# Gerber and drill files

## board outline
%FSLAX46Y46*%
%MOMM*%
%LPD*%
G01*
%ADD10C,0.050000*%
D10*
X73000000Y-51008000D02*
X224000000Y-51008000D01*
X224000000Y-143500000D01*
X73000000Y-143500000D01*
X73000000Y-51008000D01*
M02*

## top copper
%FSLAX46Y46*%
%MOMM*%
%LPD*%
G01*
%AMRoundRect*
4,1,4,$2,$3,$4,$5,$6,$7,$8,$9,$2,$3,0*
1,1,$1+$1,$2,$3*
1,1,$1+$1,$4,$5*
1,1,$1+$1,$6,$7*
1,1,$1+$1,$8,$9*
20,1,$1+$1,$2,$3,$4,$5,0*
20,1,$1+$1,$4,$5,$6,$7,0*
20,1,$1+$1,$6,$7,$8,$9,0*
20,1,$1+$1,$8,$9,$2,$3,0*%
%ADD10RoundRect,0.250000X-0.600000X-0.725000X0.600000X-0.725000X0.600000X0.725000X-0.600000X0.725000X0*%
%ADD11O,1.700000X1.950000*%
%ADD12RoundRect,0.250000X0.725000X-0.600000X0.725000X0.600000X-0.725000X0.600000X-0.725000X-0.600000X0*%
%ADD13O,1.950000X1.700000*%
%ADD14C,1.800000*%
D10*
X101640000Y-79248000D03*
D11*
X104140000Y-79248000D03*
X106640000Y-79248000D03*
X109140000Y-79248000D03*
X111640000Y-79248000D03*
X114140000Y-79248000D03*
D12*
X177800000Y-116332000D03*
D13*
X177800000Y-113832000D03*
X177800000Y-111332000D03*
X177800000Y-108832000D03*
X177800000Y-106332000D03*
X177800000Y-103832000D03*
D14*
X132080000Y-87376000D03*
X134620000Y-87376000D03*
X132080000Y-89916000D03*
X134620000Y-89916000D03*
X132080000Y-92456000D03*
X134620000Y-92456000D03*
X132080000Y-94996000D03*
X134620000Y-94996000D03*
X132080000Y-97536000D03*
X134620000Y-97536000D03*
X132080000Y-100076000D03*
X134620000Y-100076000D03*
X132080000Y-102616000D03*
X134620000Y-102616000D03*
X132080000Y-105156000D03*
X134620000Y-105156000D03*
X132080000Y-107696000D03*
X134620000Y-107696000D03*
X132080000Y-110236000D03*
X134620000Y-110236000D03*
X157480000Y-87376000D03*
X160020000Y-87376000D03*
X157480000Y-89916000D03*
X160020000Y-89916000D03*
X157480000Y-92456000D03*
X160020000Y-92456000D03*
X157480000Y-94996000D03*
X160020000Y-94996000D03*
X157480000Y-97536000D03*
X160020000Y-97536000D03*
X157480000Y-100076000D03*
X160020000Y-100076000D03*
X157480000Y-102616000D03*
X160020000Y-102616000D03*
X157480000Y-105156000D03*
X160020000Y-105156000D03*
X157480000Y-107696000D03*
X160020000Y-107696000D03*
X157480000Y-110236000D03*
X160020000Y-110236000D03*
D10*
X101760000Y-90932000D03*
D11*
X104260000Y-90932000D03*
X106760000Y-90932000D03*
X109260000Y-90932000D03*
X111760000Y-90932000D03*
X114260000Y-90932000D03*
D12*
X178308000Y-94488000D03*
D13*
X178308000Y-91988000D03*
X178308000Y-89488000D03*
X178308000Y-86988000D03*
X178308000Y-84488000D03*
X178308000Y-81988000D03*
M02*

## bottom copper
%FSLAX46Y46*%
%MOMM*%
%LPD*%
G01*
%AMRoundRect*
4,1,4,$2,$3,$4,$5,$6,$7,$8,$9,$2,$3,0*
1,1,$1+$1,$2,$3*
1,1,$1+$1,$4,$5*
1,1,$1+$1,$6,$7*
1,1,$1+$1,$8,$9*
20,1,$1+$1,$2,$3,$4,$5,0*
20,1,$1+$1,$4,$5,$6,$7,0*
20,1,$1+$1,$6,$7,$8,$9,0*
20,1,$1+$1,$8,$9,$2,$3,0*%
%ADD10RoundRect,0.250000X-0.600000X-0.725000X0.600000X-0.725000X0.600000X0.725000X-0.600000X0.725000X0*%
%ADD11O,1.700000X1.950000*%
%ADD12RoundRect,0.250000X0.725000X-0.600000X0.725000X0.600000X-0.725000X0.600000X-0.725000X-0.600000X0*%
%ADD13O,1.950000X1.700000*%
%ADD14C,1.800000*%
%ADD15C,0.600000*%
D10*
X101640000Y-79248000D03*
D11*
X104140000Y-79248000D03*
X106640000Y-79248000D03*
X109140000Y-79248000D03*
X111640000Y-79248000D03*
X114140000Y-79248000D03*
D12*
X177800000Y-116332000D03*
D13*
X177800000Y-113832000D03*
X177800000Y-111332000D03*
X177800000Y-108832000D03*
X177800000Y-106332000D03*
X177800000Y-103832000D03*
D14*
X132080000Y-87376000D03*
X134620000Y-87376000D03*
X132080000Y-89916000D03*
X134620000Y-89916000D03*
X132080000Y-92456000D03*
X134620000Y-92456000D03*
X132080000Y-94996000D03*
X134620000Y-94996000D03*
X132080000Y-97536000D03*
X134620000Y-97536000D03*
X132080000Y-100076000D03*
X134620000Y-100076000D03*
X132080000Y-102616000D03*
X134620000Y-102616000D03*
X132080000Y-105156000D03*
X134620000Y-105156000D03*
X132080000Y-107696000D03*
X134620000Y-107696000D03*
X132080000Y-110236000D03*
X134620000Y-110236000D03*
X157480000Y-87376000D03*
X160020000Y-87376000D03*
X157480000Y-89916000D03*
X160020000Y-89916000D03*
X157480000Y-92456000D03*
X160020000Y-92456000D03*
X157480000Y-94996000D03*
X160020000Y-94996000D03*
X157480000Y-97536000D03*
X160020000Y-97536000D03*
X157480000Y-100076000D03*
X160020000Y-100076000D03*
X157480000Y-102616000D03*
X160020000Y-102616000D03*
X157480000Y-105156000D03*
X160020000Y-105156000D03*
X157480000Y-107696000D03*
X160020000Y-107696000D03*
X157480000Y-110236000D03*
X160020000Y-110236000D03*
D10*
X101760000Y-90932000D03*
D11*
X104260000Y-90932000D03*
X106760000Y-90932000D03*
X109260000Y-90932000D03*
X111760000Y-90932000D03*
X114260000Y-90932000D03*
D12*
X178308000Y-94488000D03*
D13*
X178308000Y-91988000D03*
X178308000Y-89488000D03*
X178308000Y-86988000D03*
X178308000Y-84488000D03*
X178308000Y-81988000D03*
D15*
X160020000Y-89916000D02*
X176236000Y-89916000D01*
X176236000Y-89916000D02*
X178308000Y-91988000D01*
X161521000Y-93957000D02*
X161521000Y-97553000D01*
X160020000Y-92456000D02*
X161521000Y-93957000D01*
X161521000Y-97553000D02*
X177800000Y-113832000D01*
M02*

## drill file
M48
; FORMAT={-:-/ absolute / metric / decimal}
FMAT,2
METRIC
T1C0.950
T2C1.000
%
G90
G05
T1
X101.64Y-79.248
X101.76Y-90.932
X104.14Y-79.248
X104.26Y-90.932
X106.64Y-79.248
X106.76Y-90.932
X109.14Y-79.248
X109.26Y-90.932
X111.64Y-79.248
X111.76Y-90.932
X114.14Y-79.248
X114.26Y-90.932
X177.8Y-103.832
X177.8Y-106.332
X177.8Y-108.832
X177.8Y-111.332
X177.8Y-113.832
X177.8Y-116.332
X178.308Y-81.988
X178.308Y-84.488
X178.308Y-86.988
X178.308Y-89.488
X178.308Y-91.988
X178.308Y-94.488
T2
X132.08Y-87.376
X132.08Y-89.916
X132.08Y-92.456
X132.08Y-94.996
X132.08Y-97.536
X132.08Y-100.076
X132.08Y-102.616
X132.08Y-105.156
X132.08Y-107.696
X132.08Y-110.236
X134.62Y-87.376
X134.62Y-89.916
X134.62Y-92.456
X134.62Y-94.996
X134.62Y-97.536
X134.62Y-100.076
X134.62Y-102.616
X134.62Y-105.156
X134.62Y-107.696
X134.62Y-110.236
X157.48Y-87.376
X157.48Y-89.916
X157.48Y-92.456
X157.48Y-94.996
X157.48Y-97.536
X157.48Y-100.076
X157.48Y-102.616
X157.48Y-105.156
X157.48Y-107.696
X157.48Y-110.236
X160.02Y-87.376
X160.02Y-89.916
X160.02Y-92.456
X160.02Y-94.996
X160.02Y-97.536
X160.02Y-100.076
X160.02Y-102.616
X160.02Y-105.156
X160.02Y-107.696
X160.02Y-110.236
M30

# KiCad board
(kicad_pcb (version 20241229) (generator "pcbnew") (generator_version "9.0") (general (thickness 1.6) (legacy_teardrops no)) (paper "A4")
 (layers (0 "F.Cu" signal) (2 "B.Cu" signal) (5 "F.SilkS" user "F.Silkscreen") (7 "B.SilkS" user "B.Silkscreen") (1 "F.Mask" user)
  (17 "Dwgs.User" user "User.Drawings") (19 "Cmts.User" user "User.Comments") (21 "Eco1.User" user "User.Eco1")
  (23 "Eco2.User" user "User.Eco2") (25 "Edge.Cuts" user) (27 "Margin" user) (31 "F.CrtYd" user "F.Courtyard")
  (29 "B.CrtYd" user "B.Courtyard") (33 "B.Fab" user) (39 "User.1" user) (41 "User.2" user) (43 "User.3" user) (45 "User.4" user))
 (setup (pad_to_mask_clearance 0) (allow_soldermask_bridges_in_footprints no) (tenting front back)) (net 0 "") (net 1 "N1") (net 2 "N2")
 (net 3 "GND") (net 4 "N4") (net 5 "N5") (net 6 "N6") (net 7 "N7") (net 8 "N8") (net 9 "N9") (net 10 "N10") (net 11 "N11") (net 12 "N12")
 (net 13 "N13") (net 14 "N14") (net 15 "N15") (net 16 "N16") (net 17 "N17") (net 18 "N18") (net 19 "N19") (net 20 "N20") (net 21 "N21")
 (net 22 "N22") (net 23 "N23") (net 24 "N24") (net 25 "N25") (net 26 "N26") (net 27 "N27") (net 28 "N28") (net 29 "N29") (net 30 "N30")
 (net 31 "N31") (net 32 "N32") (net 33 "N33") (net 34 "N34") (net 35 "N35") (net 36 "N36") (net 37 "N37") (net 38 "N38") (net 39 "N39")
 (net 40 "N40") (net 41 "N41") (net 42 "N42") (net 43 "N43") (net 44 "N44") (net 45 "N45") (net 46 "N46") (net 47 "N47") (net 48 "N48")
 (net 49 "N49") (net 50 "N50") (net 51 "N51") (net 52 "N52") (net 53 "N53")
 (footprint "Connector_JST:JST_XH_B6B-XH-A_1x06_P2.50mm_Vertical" (layer "F.Cu") (at 101.64 79.248)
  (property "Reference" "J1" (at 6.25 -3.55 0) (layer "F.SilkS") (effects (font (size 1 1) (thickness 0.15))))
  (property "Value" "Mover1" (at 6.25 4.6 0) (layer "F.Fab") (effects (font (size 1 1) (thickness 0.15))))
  (pad "1" thru_hole roundrect (at 0 0) (size 1.7 1.95) (drill 0.95) (layers "*.Cu" "*.Mask") (remove_unused_layers no)
   (roundrect_rratio 0.147059) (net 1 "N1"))
  (pad "2" thru_hole oval (at 2.5 0) (size 1.7 1.95) (drill 0.95) (layers "*.Cu" "*.Mask") (remove_unused_layers no) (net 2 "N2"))
  (pad "3" thru_hole oval (at 5 0) (size 1.7 1.95) (drill 0.95) (layers "*.Cu" "*.Mask") (remove_unused_layers no) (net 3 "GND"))
  (pad "4" thru_hole oval (at 7.5 0) (size 1.7 1.95) (drill 0.95) (layers "*.Cu" "*.Mask") (remove_unused_layers no) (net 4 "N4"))
  (pad "5" thru_hole oval (at 10 0) (size 1.7 1.95) (drill 0.95) (layers "*.Cu" "*.Mask") (remove_unused_layers no) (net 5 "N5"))
  (pad "6" thru_hole oval (at 12.5 0) (size 1.7 1.95) (drill 0.95) (layers "*.Cu" "*.Mask") (remove_unused_layers no) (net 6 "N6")))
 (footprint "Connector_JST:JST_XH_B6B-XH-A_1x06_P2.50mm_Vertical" (layer "F.Cu") (at 177.8 116.332 90)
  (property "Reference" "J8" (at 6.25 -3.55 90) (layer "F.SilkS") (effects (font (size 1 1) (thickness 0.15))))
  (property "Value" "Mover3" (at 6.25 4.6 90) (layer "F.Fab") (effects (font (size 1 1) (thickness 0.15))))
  (pad "1" thru_hole roundrect (at 0 0 90) (size 1.7 1.95) (drill 0.95) (layers "*.Cu" "*.Mask") (remove_unused_layers no)
   (roundrect_rratio 0.147059) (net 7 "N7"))
  (pad "2" thru_hole oval (at 2.5 0 90) (size 1.7 1.95) (drill 0.95) (layers "*.Cu" "*.Mask") (remove_unused_layers no) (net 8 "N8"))
  (pad "3" thru_hole oval (at 5 0 90) (size 1.7 1.95) (drill 0.95) (layers "*.Cu" "*.Mask") (remove_unused_layers no) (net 3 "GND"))
  (pad "4" thru_hole oval (at 7.5 0 90) (size 1.7 1.95) (drill 0.95) (layers "*.Cu" "*.Mask") (remove_unused_layers no) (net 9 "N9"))
  (pad "5" thru_hole oval (at 10 0 90) (size 1.7 1.95) (drill 0.95) (layers "*.Cu" "*.Mask") (remove_unused_layers no) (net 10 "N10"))
  (pad "6" thru_hole oval (at 12.5 0 90) (size 1.7 1.95) (drill 0.95) (layers "*.Cu" "*.Mask") (remove_unused_layers no) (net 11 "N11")))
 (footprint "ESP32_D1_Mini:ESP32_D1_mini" (layer "F.Cu") (at 146.05 98.806)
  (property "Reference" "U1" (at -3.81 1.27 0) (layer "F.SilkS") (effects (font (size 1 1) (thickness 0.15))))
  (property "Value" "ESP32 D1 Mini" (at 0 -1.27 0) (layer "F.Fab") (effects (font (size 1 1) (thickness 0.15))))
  (pad "1" thru_hole circle (at -13.97 -11.43 270) (size 1.8 1.8) (drill 1) (layers "*.Cu" "*.Mask") (remove_unused_layers no)
   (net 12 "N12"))
  (pad "2" thru_hole circle (at -11.43 -11.43 270) (size 1.8 1.8) (drill 1) (layers "*.Cu" "*.Mask") (remove_unused_layers no)
   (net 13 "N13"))
  (pad "3" thru_hole circle (at -13.97 -8.89 270) (size 1.8 1.8) (drill 1) (layers "*.Cu" "*.Mask") (remove_unused_layers no) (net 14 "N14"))
  (pad "4" thru_hole circle (at -11.43 -8.89 270) (size 1.8 1.8) (drill 1) (layers "*.Cu" "*.Mask") (remove_unused_layers no) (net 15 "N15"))
  (pad "5" thru_hole circle (at -13.97 -6.35 270) (size 1.8 1.8) (drill 1) (layers "*.Cu" "*.Mask") (remove_unused_layers no) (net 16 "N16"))
  (pad "6" thru_hole circle (at -11.43 -6.35 270) (size 1.8 1.8) (drill 1) (layers "*.Cu" "*.Mask") (remove_unused_layers no) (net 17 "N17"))
  (pad "7" thru_hole circle (at -13.97 -3.81 270) (size 1.8 1.8) (drill 1) (layers "*.Cu" "*.Mask") (remove_unused_layers no) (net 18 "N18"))
  (pad "8" thru_hole circle (at -11.43 -3.81 270) (size 1.8 1.8) (drill 1) (layers "*.Cu" "*.Mask") (remove_unused_layers no) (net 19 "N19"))
  (pad "9" thru_hole circle (at -13.97 -1.27 270) (size 1.8 1.8) (drill 1) (layers "*.Cu" "*.Mask") (remove_unused_layers no) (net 7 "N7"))
  (pad "10" thru_hole circle (at -11.43 -1.27 270) (size 1.8 1.8) (drill 1) (layers "*.Cu" "*.Mask") (remove_unused_layers no)
   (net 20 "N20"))
  (pad "11" thru_hole circle (at -13.97 1.27 270) (size 1.8 1.8) (drill 1) (layers "*.Cu" "*.Mask") (remove_unused_layers no) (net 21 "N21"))
  (pad "12" thru_hole circle (at -11.43 1.27 270) (size 1.8 1.8) (drill 1) (layers "*.Cu" "*.Mask") (remove_unused_layers no) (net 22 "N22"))
  (pad "13" thru_hole circle (at -13.97 3.81 270) (size 1.8 1.8) (drill 1) (layers "*.Cu" "*.Mask") (remove_unused_layers no) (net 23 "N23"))
  (pad "14" thru_hole circle (at -11.43 3.81 270) (size 1.8 1.8) (drill 1) (layers "*.Cu" "*.Mask") (remove_unused_layers no) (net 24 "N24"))
  (pad "15" thru_hole circle (at -13.97 6.35 270) (size 1.8 1.8) (drill 1) (layers "*.Cu" "*.Mask") (remove_unused_layers no) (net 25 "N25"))
  (pad "16" thru_hole circle (at -11.43 6.35 270) (size 1.8 1.8) (drill 1) (layers "*.Cu" "*.Mask") (remove_unused_layers no) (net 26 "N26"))
  (pad "17" thru_hole circle (at -13.97 8.89 270) (size 1.8 1.8) (drill 1) (layers "*.Cu" "*.Mask") (remove_unused_layers no) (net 1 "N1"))
  (pad "18" thru_hole circle (at -11.43 8.89 270) (size 1.8 1.8) (drill 1) (layers "*.Cu" "*.Mask") (remove_unused_layers no) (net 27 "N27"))
  (pad "19" thru_hole circle (at -13.97 11.43 270) (size 1.8 1.8) (drill 1) (layers "*.Cu" "*.Mask") (remove_unused_layers no)
   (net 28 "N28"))
  (pad "20" thru_hole circle (at -11.43 11.43 270) (size 1.8 1.8) (drill 1) (layers "*.Cu" "*.Mask") (remove_unused_layers no) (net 2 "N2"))
  (pad "21" thru_hole circle (at 11.43 -11.43 270) (size 1.8 1.8) (drill 1) (layers "*.Cu" "*.Mask") (remove_unused_layers no)
   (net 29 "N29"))
  (pad "22" thru_hole circle (at 13.97 -11.43 270) (size 1.8 1.8) (drill 1) (layers "*.Cu" "*.Mask") (remove_unused_layers no)
   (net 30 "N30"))
  (pad "23" thru_hole circle (at 11.43 -8.89 270) (size 1.8 1.8) (drill 1) (layers "*.Cu" "*.Mask") (remove_unused_layers no) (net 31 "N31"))
  (pad "24" thru_hole circle (at 13.97 -8.89 270) (size 1.8 1.8) (drill 1) (layers "*.Cu" "*.Mask") (remove_unused_layers no) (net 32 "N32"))
  (pad "25" thru_hole circle (at 11.43 -6.35 270) (size 1.8 1.8) (drill 1) (layers "*.Cu" "*.Mask") (remove_unused_layers no) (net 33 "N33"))
  (pad "26" thru_hole circle (at 13.97 -6.35 270) (size 1.8 1.8) (drill 1) (layers "*.Cu" "*.Mask") (remove_unused_layers no) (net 8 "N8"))
  (pad "27" thru_hole circle (at 11.43 -3.81 270) (size 1.8 1.8) (drill 1) (layers "*.Cu" "*.Mask") (remove_unused_layers no) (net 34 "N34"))
  (pad "28" thru_hole circle (at 13.97 -3.81 270) (size 1.8 1.8) (drill 1) (layers "*.Cu" "*.Mask") (remove_unused_layers no) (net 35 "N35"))
  (pad "29" thru_hole circle (at 11.43 -1.27 270) (size 1.8 1.8) (drill 1) (layers "*.Cu" "*.Mask") (remove_unused_layers no) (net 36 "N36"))
  (pad "30" thru_hole circle (at 13.97 -1.27 270) (size 1.8 1.8) (drill 1) (layers "*.Cu" "*.Mask") (remove_unused_layers no) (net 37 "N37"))
  (pad "31" thru_hole circle (at 11.43 1.27 270) (size 1.8 1.8) (drill 1) (layers "*.Cu" "*.Mask") (remove_unused_layers no) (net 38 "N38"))
  (pad "32" thru_hole circle (at 13.97 1.27 270) (size 1.8 1.8) (drill 1) (layers "*.Cu" "*.Mask") (remove_unused_layers no) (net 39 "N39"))
  (pad "33" thru_hole circle (at 11.43 3.81 270) (size 1.8 1.8) (drill 1) (layers "*.Cu" "*.Mask") (remove_unused_layers no) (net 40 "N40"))
  (pad "34" thru_hole circle (at 13.97 3.81 270) (size 1.8 1.8) (drill 1) (layers "*.Cu" "*.Mask") (remove_unused_layers no) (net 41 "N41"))
  (pad "35" thru_hole circle (at 11.43 6.35 270) (size 1.8 1.8) (drill 1) (layers "*.Cu" "*.Mask") (remove_unused_layers no) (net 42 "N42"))
  (pad "36" thru_hole circle (at 13.97 6.35 270) (size 1.8 1.8) (drill 1) (layers "*.Cu" "*.Mask") (remove_unused_layers no) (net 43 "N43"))
  (pad "37" thru_hole circle (at 11.43 8.89 270) (size 1.8 1.8) (drill 1) (layers "*.Cu" "*.Mask") (remove_unused_layers no) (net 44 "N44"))
  (pad "38" thru_hole circle (at 13.97 8.89 270) (size 1.8 1.8) (drill 1) (layers "*.Cu" "*.Mask") (remove_unused_layers no) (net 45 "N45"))
  (pad "39" thru_hole circle (at 11.43 11.43 270) (size 1.8 1.8) (drill 1) (layers "*.Cu" "*.Mask") (remove_unused_layers no) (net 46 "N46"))
  (pad "40" thru_hole circle (at 13.97 11.43 270) (size 1.8 1.8) (drill 1) (layers "*.Cu" "*.Mask") (remove_unused_layers no) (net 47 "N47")))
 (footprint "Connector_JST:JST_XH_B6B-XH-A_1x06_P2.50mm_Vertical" (layer "F.Cu") (at 101.76 90.932)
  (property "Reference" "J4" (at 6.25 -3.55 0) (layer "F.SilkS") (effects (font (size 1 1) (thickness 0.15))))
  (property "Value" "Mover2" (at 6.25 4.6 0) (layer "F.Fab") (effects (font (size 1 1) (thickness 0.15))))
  (pad "1" thru_hole roundrect (at 0 0) (size 1.7 1.95) (drill 0.95) (layers "*.Cu" "*.Mask") (remove_unused_layers no)
   (roundrect_rratio 0.147059) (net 20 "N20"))
  (pad "2" thru_hole oval (at 2.5 0) (size 1.7 1.95) (drill 0.95) (layers "*.Cu" "*.Mask") (remove_unused_layers no) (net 35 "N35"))
  (pad "3" thru_hole oval (at 5 0) (size 1.7 1.95) (drill 0.95) (layers "*.Cu" "*.Mask") (remove_unused_layers no) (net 3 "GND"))
  (pad "4" thru_hole oval (at 7.5 0) (size 1.7 1.95) (drill 0.95) (layers "*.Cu" "*.Mask") (remove_unused_layers no) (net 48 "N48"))
  (pad "5" thru_hole oval (at 10 0) (size 1.7 1.95) (drill 0.95) (layers "*.Cu" "*.Mask") (remove_unused_layers no) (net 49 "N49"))
  (pad "6" thru_hole oval (at 12.5 0) (size 1.7 1.95) (drill 0.95) (layers "*.Cu" "*.Mask") (remove_unused_layers no) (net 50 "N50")))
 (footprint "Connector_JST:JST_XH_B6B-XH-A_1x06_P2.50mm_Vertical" (layer "F.Cu") (at 178.308 94.488 90)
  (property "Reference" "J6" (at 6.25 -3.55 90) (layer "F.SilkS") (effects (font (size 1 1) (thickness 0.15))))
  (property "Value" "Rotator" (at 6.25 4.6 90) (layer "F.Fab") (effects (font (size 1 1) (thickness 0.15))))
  (pad "1" thru_hole roundrect (at 0 0 90) (size 1.7 1.95) (drill 0.95) (layers "*.Cu" "*.Mask") (remove_unused_layers no)
   (roundrect_rratio 0.147059) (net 17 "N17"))
  (pad "2" thru_hole oval (at 2.5 0 90) (size 1.7 1.95) (drill 0.95) (layers "*.Cu" "*.Mask") (remove_unused_layers no) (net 32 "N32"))
  (pad "3" thru_hole oval (at 5 0 90) (size 1.7 1.95) (drill 0.95) (layers "*.Cu" "*.Mask") (remove_unused_layers no) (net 3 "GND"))
  (pad "4" thru_hole oval (at 7.5 0 90) (size 1.7 1.95) (drill 0.95) (layers "*.Cu" "*.Mask") (remove_unused_layers no) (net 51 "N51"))
  (pad "5" thru_hole oval (at 10 0 90) (size 1.7 1.95) (drill 0.95) (layers "*.Cu" "*.Mask") (remove_unused_layers no) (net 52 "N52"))
  (pad "6" thru_hole oval (at 12.5 0 90) (size 1.7 1.95) (drill 0.95) (layers "*.Cu" "*.Mask") (remove_unused_layers no) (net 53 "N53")))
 (gr_rect (start 73 51.008) (end 224 143.5) (stroke (width 0.05) (type default)) (fill no) (layer "Edge.Cuts"))
 (segment (start 160.02 89.916) (end 176.236 89.916) (width 0.6) (layer "B.Cu") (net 32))
 (segment (start 176.236 89.916) (end 178.308 91.988) (width 0.6) (layer "B.Cu") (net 32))
 (segment (start 161.521 93.957) (end 161.521 97.553) (width 0.6) (layer "B.Cu") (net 8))
 (segment (start 160.02 92.456) (end 161.521 93.957) (width 0.6) (layer "B.Cu") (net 8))
 (segment (start 161.521 97.553) (end 177.8 113.832) (width 0.6) (layer "B.Cu") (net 8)))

